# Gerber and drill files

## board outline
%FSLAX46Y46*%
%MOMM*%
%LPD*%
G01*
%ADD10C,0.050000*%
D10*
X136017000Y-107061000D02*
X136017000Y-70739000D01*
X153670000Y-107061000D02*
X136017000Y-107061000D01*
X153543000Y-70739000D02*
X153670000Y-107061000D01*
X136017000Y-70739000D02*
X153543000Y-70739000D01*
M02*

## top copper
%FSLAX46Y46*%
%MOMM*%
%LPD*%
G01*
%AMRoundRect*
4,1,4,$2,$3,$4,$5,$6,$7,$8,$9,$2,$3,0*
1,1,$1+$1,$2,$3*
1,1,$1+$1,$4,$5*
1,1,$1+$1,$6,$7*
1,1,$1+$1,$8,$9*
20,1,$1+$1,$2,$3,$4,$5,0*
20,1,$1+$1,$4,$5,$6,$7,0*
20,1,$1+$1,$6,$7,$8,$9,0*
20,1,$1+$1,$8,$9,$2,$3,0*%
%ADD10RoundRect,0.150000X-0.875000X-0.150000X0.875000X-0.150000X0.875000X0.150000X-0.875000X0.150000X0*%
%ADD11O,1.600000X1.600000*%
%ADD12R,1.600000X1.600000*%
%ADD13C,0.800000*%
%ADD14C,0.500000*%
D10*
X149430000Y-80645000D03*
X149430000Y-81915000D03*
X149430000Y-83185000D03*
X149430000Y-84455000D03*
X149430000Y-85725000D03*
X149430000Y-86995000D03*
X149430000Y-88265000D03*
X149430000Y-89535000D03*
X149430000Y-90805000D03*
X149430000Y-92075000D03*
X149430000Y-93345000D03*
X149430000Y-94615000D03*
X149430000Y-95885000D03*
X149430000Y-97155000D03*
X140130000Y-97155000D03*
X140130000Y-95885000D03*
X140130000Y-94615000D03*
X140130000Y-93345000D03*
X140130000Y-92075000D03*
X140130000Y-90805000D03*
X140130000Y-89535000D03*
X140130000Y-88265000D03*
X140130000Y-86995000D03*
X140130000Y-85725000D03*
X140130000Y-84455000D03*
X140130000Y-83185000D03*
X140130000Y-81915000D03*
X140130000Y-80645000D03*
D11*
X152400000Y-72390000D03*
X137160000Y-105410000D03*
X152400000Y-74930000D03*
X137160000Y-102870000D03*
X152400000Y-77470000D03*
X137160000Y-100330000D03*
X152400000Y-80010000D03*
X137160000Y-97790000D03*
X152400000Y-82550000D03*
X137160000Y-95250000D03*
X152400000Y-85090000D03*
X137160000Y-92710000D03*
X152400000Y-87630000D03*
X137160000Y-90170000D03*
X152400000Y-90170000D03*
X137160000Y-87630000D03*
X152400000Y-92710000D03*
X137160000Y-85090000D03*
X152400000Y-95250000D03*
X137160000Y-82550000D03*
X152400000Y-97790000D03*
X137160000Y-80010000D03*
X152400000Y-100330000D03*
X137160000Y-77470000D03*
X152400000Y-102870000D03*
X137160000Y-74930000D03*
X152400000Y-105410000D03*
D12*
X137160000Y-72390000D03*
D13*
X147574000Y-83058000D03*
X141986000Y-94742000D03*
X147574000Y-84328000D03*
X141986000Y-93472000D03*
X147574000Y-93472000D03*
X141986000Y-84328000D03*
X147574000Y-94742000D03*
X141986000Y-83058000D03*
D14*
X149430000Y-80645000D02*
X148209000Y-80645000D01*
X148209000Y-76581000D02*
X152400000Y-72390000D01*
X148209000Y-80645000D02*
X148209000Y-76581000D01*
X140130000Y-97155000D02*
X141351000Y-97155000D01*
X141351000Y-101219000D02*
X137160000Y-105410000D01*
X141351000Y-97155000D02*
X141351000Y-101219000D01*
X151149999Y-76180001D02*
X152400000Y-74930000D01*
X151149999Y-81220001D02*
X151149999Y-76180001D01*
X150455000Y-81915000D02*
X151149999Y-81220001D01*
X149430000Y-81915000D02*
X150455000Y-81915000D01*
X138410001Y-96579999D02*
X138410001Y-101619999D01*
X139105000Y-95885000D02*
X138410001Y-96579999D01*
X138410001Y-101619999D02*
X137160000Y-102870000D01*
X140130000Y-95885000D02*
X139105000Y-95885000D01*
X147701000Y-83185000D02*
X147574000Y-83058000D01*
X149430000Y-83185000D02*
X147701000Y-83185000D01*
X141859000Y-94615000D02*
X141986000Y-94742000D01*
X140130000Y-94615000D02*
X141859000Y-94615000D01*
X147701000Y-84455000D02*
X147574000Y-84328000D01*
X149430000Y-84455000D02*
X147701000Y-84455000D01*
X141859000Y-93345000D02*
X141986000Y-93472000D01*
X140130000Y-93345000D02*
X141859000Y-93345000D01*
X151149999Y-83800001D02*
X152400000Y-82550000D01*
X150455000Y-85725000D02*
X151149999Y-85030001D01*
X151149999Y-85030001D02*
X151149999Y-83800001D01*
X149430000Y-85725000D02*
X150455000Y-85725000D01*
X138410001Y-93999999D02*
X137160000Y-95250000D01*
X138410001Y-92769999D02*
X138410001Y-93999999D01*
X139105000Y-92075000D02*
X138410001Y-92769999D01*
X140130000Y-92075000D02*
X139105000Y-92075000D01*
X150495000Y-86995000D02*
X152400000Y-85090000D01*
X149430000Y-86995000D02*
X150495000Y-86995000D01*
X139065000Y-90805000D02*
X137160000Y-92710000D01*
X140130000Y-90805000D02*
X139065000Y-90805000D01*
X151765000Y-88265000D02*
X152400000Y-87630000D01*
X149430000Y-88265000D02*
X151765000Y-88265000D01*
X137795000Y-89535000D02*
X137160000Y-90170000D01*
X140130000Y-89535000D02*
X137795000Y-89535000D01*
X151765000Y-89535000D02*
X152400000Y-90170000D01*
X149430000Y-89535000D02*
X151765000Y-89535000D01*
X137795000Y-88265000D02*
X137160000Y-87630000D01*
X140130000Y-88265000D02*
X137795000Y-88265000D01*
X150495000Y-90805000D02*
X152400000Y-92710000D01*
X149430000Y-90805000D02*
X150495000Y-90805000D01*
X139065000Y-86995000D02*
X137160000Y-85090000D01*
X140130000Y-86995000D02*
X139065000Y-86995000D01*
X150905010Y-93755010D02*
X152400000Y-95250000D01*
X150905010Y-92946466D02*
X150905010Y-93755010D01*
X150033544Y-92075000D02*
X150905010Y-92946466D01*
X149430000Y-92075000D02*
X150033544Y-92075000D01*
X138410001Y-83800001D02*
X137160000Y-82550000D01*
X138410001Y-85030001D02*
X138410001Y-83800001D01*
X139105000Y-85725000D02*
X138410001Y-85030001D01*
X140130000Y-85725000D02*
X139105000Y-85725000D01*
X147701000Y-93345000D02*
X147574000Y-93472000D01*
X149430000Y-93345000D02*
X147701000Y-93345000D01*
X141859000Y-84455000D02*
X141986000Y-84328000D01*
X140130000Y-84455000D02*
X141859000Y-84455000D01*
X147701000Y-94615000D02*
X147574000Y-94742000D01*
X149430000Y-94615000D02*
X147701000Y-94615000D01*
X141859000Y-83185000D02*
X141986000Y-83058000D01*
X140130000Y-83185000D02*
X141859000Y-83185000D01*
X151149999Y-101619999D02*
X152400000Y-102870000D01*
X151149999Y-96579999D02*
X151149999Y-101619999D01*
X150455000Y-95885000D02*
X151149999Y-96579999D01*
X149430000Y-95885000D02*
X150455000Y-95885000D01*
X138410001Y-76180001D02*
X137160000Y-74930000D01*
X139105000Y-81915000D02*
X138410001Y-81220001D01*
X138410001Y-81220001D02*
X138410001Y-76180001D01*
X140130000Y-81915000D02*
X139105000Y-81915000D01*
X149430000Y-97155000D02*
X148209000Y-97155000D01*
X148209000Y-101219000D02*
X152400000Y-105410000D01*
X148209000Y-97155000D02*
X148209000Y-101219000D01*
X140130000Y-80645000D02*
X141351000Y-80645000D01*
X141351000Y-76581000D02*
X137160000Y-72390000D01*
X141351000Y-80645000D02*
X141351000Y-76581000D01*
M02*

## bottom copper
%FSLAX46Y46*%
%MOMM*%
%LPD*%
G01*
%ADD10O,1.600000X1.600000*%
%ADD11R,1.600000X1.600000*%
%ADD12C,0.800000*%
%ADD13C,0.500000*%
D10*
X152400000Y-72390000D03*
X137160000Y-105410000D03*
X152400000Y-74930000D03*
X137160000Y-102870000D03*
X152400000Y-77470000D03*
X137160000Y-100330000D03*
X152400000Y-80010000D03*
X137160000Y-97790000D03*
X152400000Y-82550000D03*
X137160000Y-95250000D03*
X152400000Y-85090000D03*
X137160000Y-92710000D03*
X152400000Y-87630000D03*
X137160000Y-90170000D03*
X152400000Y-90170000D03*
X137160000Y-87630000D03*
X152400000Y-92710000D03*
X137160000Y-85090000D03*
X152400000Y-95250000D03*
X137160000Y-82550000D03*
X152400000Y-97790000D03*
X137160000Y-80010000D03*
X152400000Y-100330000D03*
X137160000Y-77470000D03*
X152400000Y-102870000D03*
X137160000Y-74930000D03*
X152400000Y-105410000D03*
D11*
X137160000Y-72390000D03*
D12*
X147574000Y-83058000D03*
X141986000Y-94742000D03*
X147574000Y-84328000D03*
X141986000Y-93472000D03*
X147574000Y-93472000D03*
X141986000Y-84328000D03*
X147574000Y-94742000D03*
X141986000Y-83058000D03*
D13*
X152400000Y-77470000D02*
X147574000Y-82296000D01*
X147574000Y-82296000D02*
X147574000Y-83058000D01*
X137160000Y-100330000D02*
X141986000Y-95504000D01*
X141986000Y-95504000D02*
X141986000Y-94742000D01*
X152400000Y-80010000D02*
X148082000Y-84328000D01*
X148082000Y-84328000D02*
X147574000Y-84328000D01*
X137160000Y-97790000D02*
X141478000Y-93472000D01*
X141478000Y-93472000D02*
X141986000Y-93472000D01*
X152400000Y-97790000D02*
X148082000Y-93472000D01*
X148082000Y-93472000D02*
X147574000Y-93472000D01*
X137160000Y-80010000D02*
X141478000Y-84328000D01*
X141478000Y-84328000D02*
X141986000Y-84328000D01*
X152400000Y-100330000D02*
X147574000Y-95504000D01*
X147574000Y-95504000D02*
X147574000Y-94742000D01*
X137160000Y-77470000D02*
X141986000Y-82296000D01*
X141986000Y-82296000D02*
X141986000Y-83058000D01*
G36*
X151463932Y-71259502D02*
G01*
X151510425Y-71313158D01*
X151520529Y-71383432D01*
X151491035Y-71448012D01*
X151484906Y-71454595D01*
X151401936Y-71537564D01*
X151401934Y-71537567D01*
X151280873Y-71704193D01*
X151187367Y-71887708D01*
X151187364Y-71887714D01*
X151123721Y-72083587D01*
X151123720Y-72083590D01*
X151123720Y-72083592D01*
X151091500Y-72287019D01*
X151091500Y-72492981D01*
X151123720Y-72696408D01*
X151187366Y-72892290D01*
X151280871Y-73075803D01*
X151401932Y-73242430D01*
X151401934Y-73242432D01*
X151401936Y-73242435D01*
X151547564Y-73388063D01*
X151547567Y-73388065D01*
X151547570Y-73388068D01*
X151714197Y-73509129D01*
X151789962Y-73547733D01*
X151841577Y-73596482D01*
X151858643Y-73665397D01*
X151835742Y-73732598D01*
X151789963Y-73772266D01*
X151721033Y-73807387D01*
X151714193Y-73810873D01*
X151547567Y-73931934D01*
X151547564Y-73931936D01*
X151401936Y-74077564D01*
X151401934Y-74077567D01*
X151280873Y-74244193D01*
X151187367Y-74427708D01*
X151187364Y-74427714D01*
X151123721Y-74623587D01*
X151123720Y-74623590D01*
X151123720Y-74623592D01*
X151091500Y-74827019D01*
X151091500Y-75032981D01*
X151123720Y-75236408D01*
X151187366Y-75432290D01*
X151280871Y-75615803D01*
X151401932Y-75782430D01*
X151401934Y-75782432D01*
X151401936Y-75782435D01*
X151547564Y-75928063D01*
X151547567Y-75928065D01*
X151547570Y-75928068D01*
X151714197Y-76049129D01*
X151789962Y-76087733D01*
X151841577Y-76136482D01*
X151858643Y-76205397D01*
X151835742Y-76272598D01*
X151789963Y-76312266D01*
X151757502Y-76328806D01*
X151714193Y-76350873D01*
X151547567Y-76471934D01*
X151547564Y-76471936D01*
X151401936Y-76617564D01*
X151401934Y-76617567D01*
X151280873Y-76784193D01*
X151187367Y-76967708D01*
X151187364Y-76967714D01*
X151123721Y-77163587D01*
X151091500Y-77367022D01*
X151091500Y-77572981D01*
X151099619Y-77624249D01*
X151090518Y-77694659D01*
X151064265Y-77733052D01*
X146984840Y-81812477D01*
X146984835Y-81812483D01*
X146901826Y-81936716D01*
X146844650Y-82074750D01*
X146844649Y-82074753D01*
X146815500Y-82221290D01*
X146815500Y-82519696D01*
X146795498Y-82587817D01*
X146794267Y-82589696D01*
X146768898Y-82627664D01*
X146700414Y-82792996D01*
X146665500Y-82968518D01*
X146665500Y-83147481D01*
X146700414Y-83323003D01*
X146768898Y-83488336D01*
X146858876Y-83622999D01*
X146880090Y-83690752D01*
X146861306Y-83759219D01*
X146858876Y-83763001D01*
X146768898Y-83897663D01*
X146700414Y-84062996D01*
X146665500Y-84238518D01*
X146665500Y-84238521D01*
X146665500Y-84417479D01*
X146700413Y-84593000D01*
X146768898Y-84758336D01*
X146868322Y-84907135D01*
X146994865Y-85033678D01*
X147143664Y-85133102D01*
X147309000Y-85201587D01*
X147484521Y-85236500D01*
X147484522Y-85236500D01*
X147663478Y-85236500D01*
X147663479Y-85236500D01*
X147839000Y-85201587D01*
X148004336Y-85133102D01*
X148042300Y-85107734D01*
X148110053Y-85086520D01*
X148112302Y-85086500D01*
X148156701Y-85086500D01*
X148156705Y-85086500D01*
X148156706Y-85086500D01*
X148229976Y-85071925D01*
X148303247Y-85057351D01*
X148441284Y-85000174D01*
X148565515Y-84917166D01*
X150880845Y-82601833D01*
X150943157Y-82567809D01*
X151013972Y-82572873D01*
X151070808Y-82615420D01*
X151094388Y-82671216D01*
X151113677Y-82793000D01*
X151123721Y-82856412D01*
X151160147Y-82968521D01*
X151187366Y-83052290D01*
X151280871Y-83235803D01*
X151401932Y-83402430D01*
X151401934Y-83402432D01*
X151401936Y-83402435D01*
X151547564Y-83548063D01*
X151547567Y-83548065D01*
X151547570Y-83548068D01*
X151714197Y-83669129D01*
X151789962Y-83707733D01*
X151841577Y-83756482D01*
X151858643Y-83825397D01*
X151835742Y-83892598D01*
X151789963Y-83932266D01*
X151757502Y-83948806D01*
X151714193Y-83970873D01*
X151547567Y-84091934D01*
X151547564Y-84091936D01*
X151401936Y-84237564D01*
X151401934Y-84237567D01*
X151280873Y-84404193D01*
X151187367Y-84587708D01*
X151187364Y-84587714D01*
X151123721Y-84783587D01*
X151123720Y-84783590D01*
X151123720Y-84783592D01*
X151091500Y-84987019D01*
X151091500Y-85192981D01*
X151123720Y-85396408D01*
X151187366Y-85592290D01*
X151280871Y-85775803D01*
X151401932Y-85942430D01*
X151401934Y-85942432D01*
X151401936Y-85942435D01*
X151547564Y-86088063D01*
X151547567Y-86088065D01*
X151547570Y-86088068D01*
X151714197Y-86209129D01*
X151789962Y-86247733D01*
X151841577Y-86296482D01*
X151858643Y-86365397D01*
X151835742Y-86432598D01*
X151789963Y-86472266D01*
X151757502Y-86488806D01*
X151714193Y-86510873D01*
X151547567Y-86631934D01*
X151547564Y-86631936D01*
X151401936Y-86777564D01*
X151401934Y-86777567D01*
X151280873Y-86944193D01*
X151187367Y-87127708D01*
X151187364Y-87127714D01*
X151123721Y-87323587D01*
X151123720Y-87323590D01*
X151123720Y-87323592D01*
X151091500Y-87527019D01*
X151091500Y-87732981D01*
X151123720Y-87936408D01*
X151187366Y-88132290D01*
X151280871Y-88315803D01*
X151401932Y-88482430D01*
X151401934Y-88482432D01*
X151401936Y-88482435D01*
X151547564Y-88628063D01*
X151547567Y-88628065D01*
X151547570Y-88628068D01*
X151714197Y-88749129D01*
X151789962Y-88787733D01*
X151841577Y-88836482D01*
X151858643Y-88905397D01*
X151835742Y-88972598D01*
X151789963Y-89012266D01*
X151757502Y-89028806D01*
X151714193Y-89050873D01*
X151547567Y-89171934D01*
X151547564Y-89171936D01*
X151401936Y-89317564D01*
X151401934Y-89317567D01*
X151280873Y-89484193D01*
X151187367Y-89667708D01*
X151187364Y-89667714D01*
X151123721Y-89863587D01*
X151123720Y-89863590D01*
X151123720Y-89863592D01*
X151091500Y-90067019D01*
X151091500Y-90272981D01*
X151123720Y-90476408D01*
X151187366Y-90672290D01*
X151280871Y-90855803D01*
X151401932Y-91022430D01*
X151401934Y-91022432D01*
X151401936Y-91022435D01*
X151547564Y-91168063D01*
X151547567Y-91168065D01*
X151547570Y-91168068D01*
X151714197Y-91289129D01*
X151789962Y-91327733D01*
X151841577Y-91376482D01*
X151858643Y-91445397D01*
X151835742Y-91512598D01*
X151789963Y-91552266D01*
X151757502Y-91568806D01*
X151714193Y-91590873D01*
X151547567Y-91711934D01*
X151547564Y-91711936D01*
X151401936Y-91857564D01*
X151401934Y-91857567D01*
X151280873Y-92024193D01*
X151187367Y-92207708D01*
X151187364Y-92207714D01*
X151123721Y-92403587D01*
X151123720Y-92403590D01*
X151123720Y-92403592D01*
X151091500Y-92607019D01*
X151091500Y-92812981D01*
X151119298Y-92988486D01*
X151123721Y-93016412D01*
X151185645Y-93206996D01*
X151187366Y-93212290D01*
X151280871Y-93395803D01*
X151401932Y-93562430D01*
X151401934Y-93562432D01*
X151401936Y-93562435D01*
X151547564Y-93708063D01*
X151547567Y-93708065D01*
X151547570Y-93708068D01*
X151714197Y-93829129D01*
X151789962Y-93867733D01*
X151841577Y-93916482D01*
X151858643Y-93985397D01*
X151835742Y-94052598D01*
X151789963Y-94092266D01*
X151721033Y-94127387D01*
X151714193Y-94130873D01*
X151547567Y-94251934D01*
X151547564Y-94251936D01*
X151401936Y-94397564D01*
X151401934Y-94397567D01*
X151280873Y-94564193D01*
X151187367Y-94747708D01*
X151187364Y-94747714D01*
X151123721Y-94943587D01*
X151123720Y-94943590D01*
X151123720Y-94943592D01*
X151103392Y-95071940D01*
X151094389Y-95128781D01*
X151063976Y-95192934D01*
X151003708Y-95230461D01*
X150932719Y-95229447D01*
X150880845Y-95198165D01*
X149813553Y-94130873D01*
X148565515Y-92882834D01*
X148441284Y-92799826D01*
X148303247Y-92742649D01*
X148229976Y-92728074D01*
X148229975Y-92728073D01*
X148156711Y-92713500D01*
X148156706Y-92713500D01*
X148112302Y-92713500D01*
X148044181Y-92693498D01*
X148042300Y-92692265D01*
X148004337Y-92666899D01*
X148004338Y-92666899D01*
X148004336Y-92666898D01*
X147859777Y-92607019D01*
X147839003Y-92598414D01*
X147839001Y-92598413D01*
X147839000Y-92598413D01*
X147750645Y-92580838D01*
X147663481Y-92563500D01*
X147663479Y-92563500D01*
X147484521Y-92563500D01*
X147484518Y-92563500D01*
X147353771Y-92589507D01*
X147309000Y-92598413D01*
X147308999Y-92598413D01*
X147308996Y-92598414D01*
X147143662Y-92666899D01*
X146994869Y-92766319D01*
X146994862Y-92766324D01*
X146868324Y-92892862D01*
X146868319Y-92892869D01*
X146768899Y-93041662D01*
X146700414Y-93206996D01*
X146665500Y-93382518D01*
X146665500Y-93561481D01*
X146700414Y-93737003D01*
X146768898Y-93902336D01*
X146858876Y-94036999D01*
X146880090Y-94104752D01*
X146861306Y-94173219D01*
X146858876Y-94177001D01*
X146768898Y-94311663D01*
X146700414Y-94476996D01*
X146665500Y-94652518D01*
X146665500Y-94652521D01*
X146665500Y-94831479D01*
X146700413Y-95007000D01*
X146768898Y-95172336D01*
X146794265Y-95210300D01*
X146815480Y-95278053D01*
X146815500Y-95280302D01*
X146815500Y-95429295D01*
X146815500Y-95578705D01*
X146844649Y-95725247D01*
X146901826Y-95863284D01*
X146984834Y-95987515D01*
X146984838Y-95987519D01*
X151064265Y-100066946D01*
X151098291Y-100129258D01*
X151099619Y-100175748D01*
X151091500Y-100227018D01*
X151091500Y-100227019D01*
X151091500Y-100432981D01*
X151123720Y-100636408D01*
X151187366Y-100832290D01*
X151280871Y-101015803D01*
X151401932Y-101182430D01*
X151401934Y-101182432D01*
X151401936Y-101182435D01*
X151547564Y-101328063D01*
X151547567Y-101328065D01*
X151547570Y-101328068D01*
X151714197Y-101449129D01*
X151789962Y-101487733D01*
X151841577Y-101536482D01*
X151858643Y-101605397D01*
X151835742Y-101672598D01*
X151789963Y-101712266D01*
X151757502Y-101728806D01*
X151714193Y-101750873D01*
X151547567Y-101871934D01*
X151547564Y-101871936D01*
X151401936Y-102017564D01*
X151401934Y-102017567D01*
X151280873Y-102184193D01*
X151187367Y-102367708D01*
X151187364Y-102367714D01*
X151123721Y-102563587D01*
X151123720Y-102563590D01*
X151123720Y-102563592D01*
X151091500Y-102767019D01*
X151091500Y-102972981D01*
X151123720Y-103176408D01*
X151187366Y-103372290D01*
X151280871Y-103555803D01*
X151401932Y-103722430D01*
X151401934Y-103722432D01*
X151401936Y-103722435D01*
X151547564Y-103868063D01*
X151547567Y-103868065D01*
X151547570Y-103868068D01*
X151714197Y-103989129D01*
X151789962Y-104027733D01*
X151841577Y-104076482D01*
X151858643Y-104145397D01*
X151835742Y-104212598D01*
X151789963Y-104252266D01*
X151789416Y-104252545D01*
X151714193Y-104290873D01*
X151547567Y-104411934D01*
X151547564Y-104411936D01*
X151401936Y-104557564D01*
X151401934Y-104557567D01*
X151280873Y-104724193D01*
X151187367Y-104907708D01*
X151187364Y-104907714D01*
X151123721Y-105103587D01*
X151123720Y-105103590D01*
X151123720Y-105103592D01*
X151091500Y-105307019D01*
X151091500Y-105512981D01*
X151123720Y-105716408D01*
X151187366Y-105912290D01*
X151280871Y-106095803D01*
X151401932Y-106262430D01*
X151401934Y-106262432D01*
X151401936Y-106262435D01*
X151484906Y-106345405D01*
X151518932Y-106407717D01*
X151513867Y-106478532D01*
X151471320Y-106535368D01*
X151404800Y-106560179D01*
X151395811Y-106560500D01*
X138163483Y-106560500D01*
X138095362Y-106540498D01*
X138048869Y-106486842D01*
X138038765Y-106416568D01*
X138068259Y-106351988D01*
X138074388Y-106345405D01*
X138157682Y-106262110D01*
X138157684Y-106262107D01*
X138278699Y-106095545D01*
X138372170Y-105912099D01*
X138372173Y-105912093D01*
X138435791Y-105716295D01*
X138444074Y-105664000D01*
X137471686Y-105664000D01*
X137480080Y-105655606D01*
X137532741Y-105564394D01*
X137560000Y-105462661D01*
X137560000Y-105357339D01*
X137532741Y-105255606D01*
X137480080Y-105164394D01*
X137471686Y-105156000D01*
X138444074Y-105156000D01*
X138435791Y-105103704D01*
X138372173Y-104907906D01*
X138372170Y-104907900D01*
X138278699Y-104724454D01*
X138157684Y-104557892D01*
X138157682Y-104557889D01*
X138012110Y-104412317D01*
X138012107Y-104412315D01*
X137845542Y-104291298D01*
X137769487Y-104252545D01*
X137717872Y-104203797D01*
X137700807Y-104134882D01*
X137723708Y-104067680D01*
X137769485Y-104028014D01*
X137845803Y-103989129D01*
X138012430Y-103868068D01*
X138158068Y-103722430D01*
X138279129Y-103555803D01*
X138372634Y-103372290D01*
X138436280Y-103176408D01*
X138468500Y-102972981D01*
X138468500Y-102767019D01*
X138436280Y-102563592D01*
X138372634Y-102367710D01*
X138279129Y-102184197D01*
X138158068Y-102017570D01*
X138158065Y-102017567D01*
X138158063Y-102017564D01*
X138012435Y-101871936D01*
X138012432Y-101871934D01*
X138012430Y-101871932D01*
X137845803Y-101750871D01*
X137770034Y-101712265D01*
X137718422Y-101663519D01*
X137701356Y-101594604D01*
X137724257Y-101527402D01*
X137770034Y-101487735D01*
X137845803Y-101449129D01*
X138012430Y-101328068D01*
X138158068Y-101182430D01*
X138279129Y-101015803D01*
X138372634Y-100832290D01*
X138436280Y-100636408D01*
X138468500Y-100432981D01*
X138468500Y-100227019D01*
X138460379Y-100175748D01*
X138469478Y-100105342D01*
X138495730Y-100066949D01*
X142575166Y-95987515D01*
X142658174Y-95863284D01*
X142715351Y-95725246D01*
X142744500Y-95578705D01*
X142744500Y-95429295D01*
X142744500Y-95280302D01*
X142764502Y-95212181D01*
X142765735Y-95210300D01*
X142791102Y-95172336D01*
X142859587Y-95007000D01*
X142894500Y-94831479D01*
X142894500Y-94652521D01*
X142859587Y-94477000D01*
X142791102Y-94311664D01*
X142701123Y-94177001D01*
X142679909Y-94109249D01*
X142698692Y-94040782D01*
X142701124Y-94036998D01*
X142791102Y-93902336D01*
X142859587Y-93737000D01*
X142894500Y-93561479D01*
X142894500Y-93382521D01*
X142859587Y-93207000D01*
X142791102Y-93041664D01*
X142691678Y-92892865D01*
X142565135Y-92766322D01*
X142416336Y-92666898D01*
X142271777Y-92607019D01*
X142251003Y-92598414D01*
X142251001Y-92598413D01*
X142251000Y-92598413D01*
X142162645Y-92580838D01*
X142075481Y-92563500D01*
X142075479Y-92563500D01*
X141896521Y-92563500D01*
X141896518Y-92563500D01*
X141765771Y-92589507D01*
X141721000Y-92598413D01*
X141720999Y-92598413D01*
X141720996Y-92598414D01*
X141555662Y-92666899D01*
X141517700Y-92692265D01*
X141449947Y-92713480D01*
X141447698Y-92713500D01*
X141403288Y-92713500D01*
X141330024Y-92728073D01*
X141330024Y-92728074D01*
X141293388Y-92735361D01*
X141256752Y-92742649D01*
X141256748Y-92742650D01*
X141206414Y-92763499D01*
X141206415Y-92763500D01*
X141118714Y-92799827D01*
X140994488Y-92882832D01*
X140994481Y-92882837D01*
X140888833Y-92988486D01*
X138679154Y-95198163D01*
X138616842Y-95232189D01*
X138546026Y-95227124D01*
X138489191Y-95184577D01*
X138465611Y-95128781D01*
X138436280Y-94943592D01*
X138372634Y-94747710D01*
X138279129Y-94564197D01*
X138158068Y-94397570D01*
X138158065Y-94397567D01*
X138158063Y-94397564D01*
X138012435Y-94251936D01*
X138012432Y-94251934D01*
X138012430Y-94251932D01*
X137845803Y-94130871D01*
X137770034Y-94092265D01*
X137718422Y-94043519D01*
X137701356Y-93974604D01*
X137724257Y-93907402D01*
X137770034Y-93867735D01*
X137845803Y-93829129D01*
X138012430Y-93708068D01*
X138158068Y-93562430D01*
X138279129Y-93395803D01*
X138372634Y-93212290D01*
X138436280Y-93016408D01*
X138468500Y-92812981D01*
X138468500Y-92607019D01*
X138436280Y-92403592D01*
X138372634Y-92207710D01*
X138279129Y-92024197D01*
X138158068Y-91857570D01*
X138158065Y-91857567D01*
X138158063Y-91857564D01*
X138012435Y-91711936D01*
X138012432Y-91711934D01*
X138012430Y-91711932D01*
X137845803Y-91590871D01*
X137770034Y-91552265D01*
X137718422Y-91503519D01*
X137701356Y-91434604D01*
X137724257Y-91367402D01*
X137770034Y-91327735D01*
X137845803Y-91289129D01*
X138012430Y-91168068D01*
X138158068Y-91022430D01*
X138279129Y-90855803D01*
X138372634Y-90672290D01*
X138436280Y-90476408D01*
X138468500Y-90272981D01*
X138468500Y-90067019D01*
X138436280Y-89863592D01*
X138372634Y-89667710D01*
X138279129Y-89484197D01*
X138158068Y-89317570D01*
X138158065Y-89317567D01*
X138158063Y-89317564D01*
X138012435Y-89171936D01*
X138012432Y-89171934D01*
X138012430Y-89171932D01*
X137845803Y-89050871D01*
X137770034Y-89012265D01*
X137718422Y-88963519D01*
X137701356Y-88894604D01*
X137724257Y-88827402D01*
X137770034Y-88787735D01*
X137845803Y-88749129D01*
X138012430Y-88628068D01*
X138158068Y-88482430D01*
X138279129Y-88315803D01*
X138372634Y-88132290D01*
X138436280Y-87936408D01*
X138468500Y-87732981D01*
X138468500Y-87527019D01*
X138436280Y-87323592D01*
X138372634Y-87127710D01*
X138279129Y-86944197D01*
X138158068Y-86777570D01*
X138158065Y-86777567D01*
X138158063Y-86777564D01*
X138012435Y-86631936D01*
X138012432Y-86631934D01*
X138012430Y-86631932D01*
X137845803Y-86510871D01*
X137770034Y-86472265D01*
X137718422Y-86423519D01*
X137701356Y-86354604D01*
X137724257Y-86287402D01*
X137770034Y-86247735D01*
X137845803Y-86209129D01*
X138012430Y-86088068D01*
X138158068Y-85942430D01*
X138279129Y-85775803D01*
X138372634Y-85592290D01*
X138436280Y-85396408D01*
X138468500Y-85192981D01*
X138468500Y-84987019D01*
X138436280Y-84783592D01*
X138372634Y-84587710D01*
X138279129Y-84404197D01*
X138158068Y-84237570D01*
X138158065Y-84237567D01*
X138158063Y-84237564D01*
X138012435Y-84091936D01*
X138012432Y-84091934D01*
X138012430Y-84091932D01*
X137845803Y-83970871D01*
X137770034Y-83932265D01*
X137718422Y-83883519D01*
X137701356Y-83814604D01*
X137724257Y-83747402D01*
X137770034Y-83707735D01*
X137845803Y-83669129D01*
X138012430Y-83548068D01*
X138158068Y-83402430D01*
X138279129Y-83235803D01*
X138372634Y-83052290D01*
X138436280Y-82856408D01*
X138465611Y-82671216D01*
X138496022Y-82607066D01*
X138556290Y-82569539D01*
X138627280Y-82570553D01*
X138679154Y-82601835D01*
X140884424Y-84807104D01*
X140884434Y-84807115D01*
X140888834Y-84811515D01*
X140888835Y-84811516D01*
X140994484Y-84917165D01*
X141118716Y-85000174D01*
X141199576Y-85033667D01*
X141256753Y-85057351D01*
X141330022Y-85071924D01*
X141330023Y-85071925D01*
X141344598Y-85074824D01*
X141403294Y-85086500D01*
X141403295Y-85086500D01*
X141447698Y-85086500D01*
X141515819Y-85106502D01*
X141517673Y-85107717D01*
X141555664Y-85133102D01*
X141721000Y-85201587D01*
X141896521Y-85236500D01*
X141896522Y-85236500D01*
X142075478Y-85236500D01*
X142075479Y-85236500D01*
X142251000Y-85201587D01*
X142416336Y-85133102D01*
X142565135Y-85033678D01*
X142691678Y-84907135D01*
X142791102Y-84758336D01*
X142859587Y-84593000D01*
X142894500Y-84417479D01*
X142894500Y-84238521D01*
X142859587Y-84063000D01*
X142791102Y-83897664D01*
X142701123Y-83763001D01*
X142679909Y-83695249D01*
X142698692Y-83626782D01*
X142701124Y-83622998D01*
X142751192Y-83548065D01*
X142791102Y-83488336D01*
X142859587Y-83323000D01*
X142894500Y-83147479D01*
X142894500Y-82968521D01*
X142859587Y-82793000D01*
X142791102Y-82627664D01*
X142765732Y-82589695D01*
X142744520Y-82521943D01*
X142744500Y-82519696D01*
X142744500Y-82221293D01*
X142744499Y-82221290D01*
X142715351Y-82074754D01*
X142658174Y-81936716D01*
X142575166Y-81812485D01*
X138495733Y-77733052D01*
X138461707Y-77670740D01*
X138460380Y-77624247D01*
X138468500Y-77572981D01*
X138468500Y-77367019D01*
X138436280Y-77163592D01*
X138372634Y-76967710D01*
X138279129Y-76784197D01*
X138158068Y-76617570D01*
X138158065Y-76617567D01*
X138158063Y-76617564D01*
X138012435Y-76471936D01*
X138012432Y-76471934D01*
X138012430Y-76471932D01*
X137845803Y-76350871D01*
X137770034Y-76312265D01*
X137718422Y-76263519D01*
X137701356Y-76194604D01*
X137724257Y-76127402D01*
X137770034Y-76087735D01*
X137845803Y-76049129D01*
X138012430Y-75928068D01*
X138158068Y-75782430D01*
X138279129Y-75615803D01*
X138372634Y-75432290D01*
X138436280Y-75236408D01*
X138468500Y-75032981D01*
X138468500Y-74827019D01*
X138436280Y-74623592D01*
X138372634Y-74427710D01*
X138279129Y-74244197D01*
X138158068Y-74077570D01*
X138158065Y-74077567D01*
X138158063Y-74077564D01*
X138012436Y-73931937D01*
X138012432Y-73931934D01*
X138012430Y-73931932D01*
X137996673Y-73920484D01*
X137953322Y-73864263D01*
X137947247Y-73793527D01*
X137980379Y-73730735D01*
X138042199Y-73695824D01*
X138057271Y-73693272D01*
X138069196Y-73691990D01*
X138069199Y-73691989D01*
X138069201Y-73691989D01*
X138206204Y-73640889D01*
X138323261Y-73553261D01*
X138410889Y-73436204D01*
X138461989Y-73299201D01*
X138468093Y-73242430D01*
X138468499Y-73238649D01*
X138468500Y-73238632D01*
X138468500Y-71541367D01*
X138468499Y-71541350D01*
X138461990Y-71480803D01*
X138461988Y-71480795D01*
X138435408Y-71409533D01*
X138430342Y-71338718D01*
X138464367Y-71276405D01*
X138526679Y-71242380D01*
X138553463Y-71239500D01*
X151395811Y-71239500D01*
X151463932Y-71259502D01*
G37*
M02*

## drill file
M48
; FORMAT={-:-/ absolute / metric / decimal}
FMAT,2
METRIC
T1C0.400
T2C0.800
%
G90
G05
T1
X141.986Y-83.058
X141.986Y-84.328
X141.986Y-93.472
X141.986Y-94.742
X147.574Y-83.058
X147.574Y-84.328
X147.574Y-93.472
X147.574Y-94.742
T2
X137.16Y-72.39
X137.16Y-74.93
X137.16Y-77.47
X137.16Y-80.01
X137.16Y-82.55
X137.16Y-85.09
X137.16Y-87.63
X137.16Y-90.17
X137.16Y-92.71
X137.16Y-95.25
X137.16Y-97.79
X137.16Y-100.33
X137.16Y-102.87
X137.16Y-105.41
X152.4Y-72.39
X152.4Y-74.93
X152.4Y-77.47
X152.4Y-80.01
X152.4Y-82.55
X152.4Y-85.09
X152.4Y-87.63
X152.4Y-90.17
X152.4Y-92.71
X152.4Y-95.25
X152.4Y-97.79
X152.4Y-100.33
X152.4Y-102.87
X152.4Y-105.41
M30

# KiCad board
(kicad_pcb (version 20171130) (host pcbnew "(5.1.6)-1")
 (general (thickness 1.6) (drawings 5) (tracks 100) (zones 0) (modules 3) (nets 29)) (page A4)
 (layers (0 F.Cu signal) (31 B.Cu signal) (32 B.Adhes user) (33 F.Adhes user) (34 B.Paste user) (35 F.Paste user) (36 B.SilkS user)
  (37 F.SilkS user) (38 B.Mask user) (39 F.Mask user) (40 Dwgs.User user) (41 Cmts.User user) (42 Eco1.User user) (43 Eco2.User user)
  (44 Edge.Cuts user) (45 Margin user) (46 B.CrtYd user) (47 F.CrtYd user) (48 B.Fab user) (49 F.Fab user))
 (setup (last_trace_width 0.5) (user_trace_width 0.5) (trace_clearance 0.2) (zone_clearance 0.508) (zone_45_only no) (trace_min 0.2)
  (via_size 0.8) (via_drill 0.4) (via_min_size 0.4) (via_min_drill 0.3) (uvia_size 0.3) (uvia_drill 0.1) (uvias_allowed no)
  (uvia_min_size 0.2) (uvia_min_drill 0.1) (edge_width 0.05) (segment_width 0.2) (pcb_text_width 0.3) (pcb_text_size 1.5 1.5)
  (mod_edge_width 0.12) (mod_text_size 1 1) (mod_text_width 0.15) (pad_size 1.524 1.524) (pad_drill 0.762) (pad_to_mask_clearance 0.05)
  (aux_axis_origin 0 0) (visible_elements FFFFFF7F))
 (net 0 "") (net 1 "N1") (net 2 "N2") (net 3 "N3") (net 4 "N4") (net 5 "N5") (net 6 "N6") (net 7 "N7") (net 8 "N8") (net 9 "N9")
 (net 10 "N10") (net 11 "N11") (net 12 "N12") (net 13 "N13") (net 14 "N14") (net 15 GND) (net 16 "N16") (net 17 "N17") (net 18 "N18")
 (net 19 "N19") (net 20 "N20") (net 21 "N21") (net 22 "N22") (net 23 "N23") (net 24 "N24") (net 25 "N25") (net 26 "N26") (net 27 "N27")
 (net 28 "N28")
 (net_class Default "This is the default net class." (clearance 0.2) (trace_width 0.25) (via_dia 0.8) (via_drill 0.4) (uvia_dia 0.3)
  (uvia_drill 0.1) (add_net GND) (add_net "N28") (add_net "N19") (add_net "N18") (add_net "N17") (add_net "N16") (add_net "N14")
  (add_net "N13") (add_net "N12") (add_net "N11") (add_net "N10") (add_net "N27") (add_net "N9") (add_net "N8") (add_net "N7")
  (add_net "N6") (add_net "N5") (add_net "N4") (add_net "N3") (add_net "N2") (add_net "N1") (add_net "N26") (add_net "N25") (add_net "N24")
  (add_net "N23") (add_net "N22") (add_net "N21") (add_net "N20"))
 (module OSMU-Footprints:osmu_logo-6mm (layer F.Cu) (at 144.78 74.549)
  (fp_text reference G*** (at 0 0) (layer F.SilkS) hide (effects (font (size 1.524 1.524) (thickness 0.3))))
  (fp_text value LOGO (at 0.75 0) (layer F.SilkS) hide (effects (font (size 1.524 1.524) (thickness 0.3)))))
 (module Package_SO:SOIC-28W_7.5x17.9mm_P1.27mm (layer F.Cu) (at 144.78 88.9)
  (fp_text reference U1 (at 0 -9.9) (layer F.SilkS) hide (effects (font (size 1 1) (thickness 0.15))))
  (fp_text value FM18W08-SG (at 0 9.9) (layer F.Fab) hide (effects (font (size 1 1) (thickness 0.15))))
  (pad 28 smd roundrect (at 4.65 -8.255) (size 2.05 0.6) (layers F.Cu F.Paste F.Mask) (roundrect_rratio 0.25) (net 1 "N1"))
  (pad 27 smd roundrect (at 4.65 -6.985) (size 2.05 0.6) (layers F.Cu F.Paste F.Mask) (roundrect_rratio 0.25) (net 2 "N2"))
  (pad 26 smd roundrect (at 4.65 -5.715) (size 2.05 0.6) (layers F.Cu F.Paste F.Mask) (roundrect_rratio 0.25) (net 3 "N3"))
  (pad 25 smd roundrect (at 4.65 -4.445) (size 2.05 0.6) (layers F.Cu F.Paste F.Mask) (roundrect_rratio 0.25) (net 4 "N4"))
  (pad 24 smd roundrect (at 4.65 -3.175) (size 2.05 0.6) (layers F.Cu F.Paste F.Mask) (roundrect_rratio 0.25) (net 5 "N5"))
  (pad 23 smd roundrect (at 4.65 -1.905) (size 2.05 0.6) (layers F.Cu F.Paste F.Mask) (roundrect_rratio 0.25) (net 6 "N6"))
  (pad 22 smd roundrect (at 4.65 -0.635) (size 2.05 0.6) (layers F.Cu F.Paste F.Mask) (roundrect_rratio 0.25) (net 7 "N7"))
  (pad 21 smd roundrect (at 4.65 0.635) (size 2.05 0.6) (layers F.Cu F.Paste F.Mask) (roundrect_rratio 0.25) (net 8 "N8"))
  (pad 20 smd roundrect (at 4.65 1.905) (size 2.05 0.6) (layers F.Cu F.Paste F.Mask) (roundrect_rratio 0.25) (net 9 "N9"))
  (pad 19 smd roundrect (at 4.65 3.175) (size 2.05 0.6) (layers F.Cu F.Paste F.Mask) (roundrect_rratio 0.25) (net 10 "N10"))
  (pad 18 smd roundrect (at 4.65 4.445) (size 2.05 0.6) (layers F.Cu F.Paste F.Mask) (roundrect_rratio 0.25) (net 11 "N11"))
  (pad 17 smd roundrect (at 4.65 5.715) (size 2.05 0.6) (layers F.Cu F.Paste F.Mask) (roundrect_rratio 0.25) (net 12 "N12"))
  (pad 16 smd roundrect (at 4.65 6.985) (size 2.05 0.6) (layers F.Cu F.Paste F.Mask) (roundrect_rratio 0.25) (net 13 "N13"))
  (pad 15 smd roundrect (at 4.65 8.255) (size 2.05 0.6) (layers F.Cu F.Paste F.Mask) (roundrect_rratio 0.25) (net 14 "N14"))
  (pad 14 smd roundrect (at -4.65 8.255) (size 2.05 0.6) (layers F.Cu F.Paste F.Mask) (roundrect_rratio 0.25) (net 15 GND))
  (pad 13 smd roundrect (at -4.65 6.985) (size 2.05 0.6) (layers F.Cu F.Paste F.Mask) (roundrect_rratio 0.25) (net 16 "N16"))
  (pad 12 smd roundrect (at -4.65 5.715) (size 2.05 0.6) (layers F.Cu F.Paste F.Mask) (roundrect_rratio 0.25) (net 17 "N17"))
  (pad 11 smd roundrect (at -4.65 4.445) (size 2.05 0.6) (layers F.Cu F.Paste F.Mask) (roundrect_rratio 0.25) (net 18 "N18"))
  (pad 10 smd roundrect (at -4.65 3.175) (size 2.05 0.6) (layers F.Cu F.Paste F.Mask) (roundrect_rratio 0.25) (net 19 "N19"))
  (pad 9 smd roundrect (at -4.65 1.905) (size 2.05 0.6) (layers F.Cu F.Paste F.Mask) (roundrect_rratio 0.25) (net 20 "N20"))
  (pad 8 smd roundrect (at -4.65 0.635) (size 2.05 0.6) (layers F.Cu F.Paste F.Mask) (roundrect_rratio 0.25) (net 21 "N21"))
  (pad 7 smd roundrect (at -4.65 -0.635) (size 2.05 0.6) (layers F.Cu F.Paste F.Mask) (roundrect_rratio 0.25) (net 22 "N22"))
  (pad 6 smd roundrect (at -4.65 -1.905) (size 2.05 0.6) (layers F.Cu F.Paste F.Mask) (roundrect_rratio 0.25) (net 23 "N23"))
  (pad 5 smd roundrect (at -4.65 -3.175) (size 2.05 0.6) (layers F.Cu F.Paste F.Mask) (roundrect_rratio 0.25) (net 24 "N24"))
  (pad 4 smd roundrect (at -4.65 -4.445) (size 2.05 0.6) (layers F.Cu F.Paste F.Mask) (roundrect_rratio 0.25) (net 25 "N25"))
  (pad 3 smd roundrect (at -4.65 -5.715) (size 2.05 0.6) (layers F.Cu F.Paste F.Mask) (roundrect_rratio 0.25) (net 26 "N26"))
  (pad 2 smd roundrect (at -4.65 -6.985) (size 2.05 0.6) (layers F.Cu F.Paste F.Mask) (roundrect_rratio 0.25) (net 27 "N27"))
  (pad 1 smd roundrect (at -4.65 -8.255) (size 2.05 0.6) (layers F.Cu F.Paste F.Mask) (roundrect_rratio 0.25) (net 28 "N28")))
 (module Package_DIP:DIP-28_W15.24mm (layer F.Cu) (at 137.16 72.39)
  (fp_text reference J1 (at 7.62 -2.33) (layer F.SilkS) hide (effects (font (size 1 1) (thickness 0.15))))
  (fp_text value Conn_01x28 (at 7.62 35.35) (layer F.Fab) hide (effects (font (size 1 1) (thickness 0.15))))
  (pad 28 thru_hole oval (at 15.24 0) (size 1.6 1.6) (drill 0.8) (layers *.Cu *.Mask) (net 1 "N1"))
  (pad 14 thru_hole oval (at 0 33.02) (size 1.6 1.6) (drill 0.8) (layers *.Cu *.Mask) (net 15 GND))
  (pad 27 thru_hole oval (at 15.24 2.54) (size 1.6 1.6) (drill 0.8) (layers *.Cu *.Mask) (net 2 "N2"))
  (pad 13 thru_hole oval (at 0 30.48) (size 1.6 1.6) (drill 0.8) (layers *.Cu *.Mask) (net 16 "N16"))
  (pad 26 thru_hole oval (at 15.24 5.08) (size 1.6 1.6) (drill 0.8) (layers *.Cu *.Mask) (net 3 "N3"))
  (pad 12 thru_hole oval (at 0 27.94) (size 1.6 1.6) (drill 0.8) (layers *.Cu *.Mask) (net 17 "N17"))
  (pad 25 thru_hole oval (at 15.24 7.62) (size 1.6 1.6) (drill 0.8) (layers *.Cu *.Mask) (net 4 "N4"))
  (pad 11 thru_hole oval (at 0 25.4) (size 1.6 1.6) (drill 0.8) (layers *.Cu *.Mask) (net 18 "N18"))
  (pad 24 thru_hole oval (at 15.24 10.16) (size 1.6 1.6) (drill 0.8) (layers *.Cu *.Mask) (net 5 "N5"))
  (pad 10 thru_hole oval (at 0 22.86) (size 1.6 1.6) (drill 0.8) (layers *.Cu *.Mask) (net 19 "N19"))
  (pad 23 thru_hole oval (at 15.24 12.7) (size 1.6 1.6) (drill 0.8) (layers *.Cu *.Mask) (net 6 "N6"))
  (pad 9 thru_hole oval (at 0 20.32) (size 1.6 1.6) (drill 0.8) (layers *.Cu *.Mask) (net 20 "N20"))
  (pad 22 thru_hole oval (at 15.24 15.24) (size 1.6 1.6) (drill 0.8) (layers *.Cu *.Mask) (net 7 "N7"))
  (pad 8 thru_hole oval (at 0 17.78) (size 1.6 1.6) (drill 0.8) (layers *.Cu *.Mask) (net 21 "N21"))
  (pad 21 thru_hole oval (at 15.24 17.78) (size 1.6 1.6) (drill 0.8) (layers *.Cu *.Mask) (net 8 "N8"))
  (pad 7 thru_hole oval (at 0 15.24) (size 1.6 1.6) (drill 0.8) (layers *.Cu *.Mask) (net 22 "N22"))
  (pad 20 thru_hole oval (at 15.24 20.32) (size 1.6 1.6) (drill 0.8) (layers *.Cu *.Mask) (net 9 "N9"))
  (pad 6 thru_hole oval (at 0 12.7) (size 1.6 1.6) (drill 0.8) (layers *.Cu *.Mask) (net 23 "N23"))
  (pad 19 thru_hole oval (at 15.24 22.86) (size 1.6 1.6) (drill 0.8) (layers *.Cu *.Mask) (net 10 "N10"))
  (pad 5 thru_hole oval (at 0 10.16) (size 1.6 1.6) (drill 0.8) (layers *.Cu *.Mask) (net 24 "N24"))
  (pad 18 thru_hole oval (at 15.24 25.4) (size 1.6 1.6) (drill 0.8) (layers *.Cu *.Mask) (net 11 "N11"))
  (pad 4 thru_hole oval (at 0 7.62) (size 1.6 1.6) (drill 0.8) (layers *.Cu *.Mask) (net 25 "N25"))
  (pad 17 thru_hole oval (at 15.24 27.94) (size 1.6 1.6) (drill 0.8) (layers *.Cu *.Mask) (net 12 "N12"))
  (pad 3 thru_hole oval (at 0 5.08) (size 1.6 1.6) (drill 0.8) (layers *.Cu *.Mask) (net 26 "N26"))
  (pad 16 thru_hole oval (at 15.24 30.48) (size 1.6 1.6) (drill 0.8) (layers *.Cu *.Mask) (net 13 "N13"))
  (pad 2 thru_hole oval (at 0 2.54) (size 1.6 1.6) (drill 0.8) (layers *.Cu *.Mask) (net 27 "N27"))
  (pad 15 thru_hole oval (at 15.24 33.02) (size 1.6 1.6) (drill 0.8) (layers *.Cu *.Mask) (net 14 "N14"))
  (pad 1 thru_hole rect (at 0 0) (size 1.6 1.6) (drill 0.8) (layers *.Cu *.Mask) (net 28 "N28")))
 (gr_line (start 136.017 107.061) (end 136.017 70.739) (layer Edge.Cuts) (width 0.05))
 (gr_line (start 153.67 107.061) (end 136.017 107.061) (layer Edge.Cuts) (width 0.05))
 (gr_line (start 153.543 70.739) (end 153.67 107.061) (layer Edge.Cuts) (width 0.05))
 (gr_line (start 136.017 70.739) (end 153.543 70.739) (layer Edge.Cuts) (width 0.05))
 (segment (start 149.43 80.645) (end 148.209 80.645) (width 0.5) (layer F.Cu) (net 1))
 (segment (start 148.209 76.581) (end 152.4 72.39) (width 0.5) (layer F.Cu) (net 1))
 (segment (start 148.209 80.645) (end 148.209 76.581) (width 0.5) (layer F.Cu) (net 1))
 (segment (start 140.13 97.155) (end 141.351 97.155) (width 0.5) (layer F.Cu) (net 15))
 (segment (start 141.351 101.219) (end 137.16 105.41) (width 0.5) (layer F.Cu) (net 15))
 (segment (start 141.351 97.155) (end 141.351 101.219) (width 0.5) (layer F.Cu) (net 15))
 (segment (start 151.149999 76.180001) (end 152.4 74.93) (width 0.5) (layer F.Cu) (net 2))
 (segment (start 151.149999 81.220001) (end 151.149999 76.180001) (width 0.5) (layer F.Cu) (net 2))
 (segment (start 150.455 81.915) (end 151.149999 81.220001) (width 0.5) (layer F.Cu) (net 2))
 (segment (start 149.43 81.915) (end 150.455 81.915) (width 0.5) (layer F.Cu) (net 2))
 (segment (start 138.410001 96.579999) (end 138.410001 101.619999) (width 0.5) (layer F.Cu) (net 16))
 (segment (start 139.105 95.885) (end 138.410001 96.579999) (width 0.5) (layer F.Cu) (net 16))
 (segment (start 138.410001 101.619999) (end 137.16 102.87) (width 0.5) (layer F.Cu) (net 16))
 (segment (start 140.13 95.885) (end 139.105 95.885) (width 0.5) (layer F.Cu) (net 16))
 (via (at 147.574 83.058) (size 0.8) (drill 0.4) (layers F.Cu B.Cu) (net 3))
 (segment (start 152.4 77.47) (end 147.574 82.296) (width 0.5) (layer B.Cu) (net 3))
 (segment (start 147.574 82.296) (end 147.574 83.058) (width 0.5) (layer B.Cu) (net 3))
 (segment (start 147.701 83.185) (end 147.574 83.058) (width 0.5) (layer F.Cu) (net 3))
 (segment (start 149.43 83.185) (end 147.701 83.185) (width 0.5) (layer F.Cu) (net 3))
 (via (at 141.986 94.742) (size 0.8) (drill 0.4) (layers F.Cu B.Cu) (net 17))
 (segment (start 137.16 100.33) (end 141.986 95.504) (width 0.5) (layer B.Cu) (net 17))
 (segment (start 141.986 95.504) (end 141.986 94.742) (width 0.5) (layer B.Cu) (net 17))
 (segment (start 141.859 94.615) (end 141.986 94.742) (width 0.5) (layer F.Cu) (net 17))
 (segment (start 140.13 94.615) (end 141.859 94.615) (width 0.5) (layer F.Cu) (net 17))
 (via (at 147.574 84.328) (size 0.8) (drill 0.4) (layers F.Cu B.Cu) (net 4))
 (segment (start 152.4 80.01) (end 148.082 84.328) (width 0.5) (layer B.Cu) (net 4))
 (segment (start 147.701 84.455) (end 147.574 84.328) (width 0.5) (layer F.Cu) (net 4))
 (segment (start 149.43 84.455) (end 147.701 84.455) (width 0.5) (layer F.Cu) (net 4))
 (segment (start 148.082 84.328) (end 147.574 84.328) (width 0.5) (layer B.Cu) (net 4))
 (via (at 141.986 93.472) (size 0.8) (drill 0.4) (layers F.Cu B.Cu) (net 18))
 (segment (start 137.16 97.79) (end 141.478 93.472) (width 0.5) (layer B.Cu) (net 18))
 (segment (start 141.478 93.472) (end 141.986 93.472) (width 0.5) (layer B.Cu) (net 18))
 (segment (start 141.859 93.345) (end 141.986 93.472) (width 0.5) (layer F.Cu) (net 18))
 (segment (start 140.13 93.345) (end 141.859 93.345) (width 0.5) (layer F.Cu) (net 18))
 (segment (start 151.149999 83.800001) (end 152.4 82.55) (width 0.5) (layer F.Cu) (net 5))
 (segment (start 150.455 85.725) (end 151.149999 85.030001) (width 0.5) (layer F.Cu) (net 5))
 (segment (start 151.149999 85.030001) (end 151.149999 83.800001) (width 0.5) (layer F.Cu) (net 5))
 (segment (start 149.43 85.725) (end 150.455 85.725) (width 0.5) (layer F.Cu) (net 5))
 (segment (start 138.410001 93.999999) (end 137.16 95.25) (width 0.5) (layer F.Cu) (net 19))
 (segment (start 138.410001 92.769999) (end 138.410001 93.999999) (width 0.5) (layer F.Cu) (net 19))
 (segment (start 139.105 92.075) (end 138.410001 92.769999) (width 0.5) (layer F.Cu) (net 19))
 (segment (start 140.13 92.075) (end 139.105 92.075) (width 0.5) (layer F.Cu) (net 19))
 (segment (start 150.495 86.995) (end 152.4 85.09) (width 0.5) (layer F.Cu) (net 6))
 (segment (start 149.43 86.995) (end 150.495 86.995) (width 0.5) (layer F.Cu) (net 6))
 (segment (start 139.065 90.805) (end 137.16 92.71) (width 0.5) (layer F.Cu) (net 20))
 (segment (start 140.13 90.805) (end 139.065 90.805) (width 0.5) (layer F.Cu) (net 20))
 (segment (start 151.765 88.265) (end 152.4 87.63) (width 0.5) (layer F.Cu) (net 7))
 (segment (start 149.43 88.265) (end 151.765 88.265) (width 0.5) (layer F.Cu) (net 7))
 (segment (start 137.795 89.535) (end 137.16 90.17) (width 0.5) (layer F.Cu) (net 21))
 (segment (start 140.13 89.535) (end 137.795 89.535) (width 0.5) (layer F.Cu) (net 21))
 (segment (start 151.765 89.535) (end 152.4 90.17) (width 0.5) (layer F.Cu) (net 8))
 (segment (start 149.43 89.535) (end 151.765 89.535) (width 0.5) (layer F.Cu) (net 8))
 (segment (start 137.795 88.265) (end 137.16 87.63) (width 0.5) (layer F.Cu) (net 22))
 (segment (start 140.13 88.265) (end 137.795 88.265) (width 0.5) (layer F.Cu) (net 22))
 (segment (start 150.495 90.805) (end 152.4 92.71) (width 0.5) (layer F.Cu) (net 9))
 (segment (start 149.43 90.805) (end 150.495 90.805) (width 0.5) (layer F.Cu) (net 9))
 (segment (start 139.065 86.995) (end 137.16 85.09) (width 0.5) (layer F.Cu) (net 23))
 (segment (start 140.13 86.995) (end 139.065 86.995) (width 0.5) (layer F.Cu) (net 23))
 (segment (start 150.90501 93.75501) (end 152.4 95.25) (width 0.5) (layer F.Cu) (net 10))
 (segment (start 150.90501 92.946466) (end 150.90501 93.75501) (width 0.5) (layer F.Cu) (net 10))
 (segment (start 150.033544 92.075) (end 150.90501 92.946466) (width 0.5) (layer F.Cu) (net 10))
 (segment (start 149.43 92.075) (end 150.033544 92.075) (width 0.5) (layer F.Cu) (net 10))
 (segment (start 138.410001 83.800001) (end 137.16 82.55) (width 0.5) (layer F.Cu) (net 24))
 (segment (start 138.410001 85.030001) (end 138.410001 83.800001) (width 0.5) (layer F.Cu) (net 24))
 (segment (start 139.105 85.725) (end 138.410001 85.030001) (width 0.5) (layer F.Cu) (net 24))
 (segment (start 140.13 85.725) (end 139.105 85.725) (width 0.5) (layer F.Cu) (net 24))
 (via (at 147.574 93.472) (size 0.8) (drill 0.4) (layers F.Cu B.Cu) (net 11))
 (segment (start 152.4 97.79) (end 148.082 93.472) (width 0.5) (layer B.Cu) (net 11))
 (segment (start 148.082 93.472) (end 147.574 93.472) (width 0.5) (layer B.Cu) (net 11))
 (segment (start 147.701 93.345) (end 147.574 93.472) (width 0.5) (layer F.Cu) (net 11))
 (segment (start 149.43 93.345) (end 147.701 93.345) (width 0.5) (layer F.Cu) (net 11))
 (via (at 141.986 84.328) (size 0.8) (drill 0.4) (layers F.Cu B.Cu) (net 25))
 (segment (start 137.16 80.01) (end 141.478 84.328) (width 0.5) (layer B.Cu) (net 25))
 (segment (start 141.478 84.328) (end 141.986 84.328) (width 0.5) (layer B.Cu) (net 25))
 (segment (start 141.859 84.455) (end 141.986 84.328) (width 0.5) (layer F.Cu) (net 25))
 (segment (start 140.13 84.455) (end 141.859 84.455) (width 0.5) (layer F.Cu) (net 25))
 (via (at 147.574 94.742) (size 0.8) (drill 0.4) (layers F.Cu B.Cu) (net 12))
 (segment (start 152.4 100.33) (end 147.574 95.504) (width 0.5) (layer B.Cu) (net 12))
 (segment (start 147.574 95.504) (end 147.574 94.742) (width 0.5) (layer B.Cu) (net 12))
 (segment (start 147.701 94.615) (end 147.574 94.742) (width 0.5) (layer F.Cu) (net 12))
 (segment (start 149.43 94.615) (end 147.701 94.615) (width 0.5) (layer F.Cu) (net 12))
 (via (at 141.986 83.058) (size 0.8) (drill 0.4) (layers F.Cu B.Cu) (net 26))
 (segment (start 137.16 77.47) (end 141.986 82.296) (width 0.5) (layer B.Cu) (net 26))
 (segment (start 141.986 82.296) (end 141.986 83.058) (width 0.5) (layer B.Cu) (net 26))
 (segment (start 141.859 83.185) (end 141.986 83.058) (width 0.5) (layer F.Cu) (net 26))
 (segment (start 140.13 83.185) (end 141.859 83.185) (width 0.5) (layer F.Cu) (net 26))
 (segment (start 151.149999 101.619999) (end 152.4 102.87) (width 0.5) (layer F.Cu) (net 13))
 (segment (start 151.149999 96.579999) (end 151.149999 101.619999) (width 0.5) (layer F.Cu) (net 13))
 (segment (start 150.455 95.885) (end 151.149999 96.579999) (width 0.5) (layer F.Cu) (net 13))
 (segment (start 149.43 95.885) (end 150.455 95.885) (width 0.5) (layer F.Cu) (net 13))
 (segment (start 138.410001 76.180001) (end 137.16 74.93) (width 0.5) (layer F.Cu) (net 27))
 (segment (start 139.105 81.915) (end 138.410001 81.220001) (width 0.5) (layer F.Cu) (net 27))
 (segment (start 138.410001 81.220001) (end 138.410001 76.180001) (width 0.5) (layer F.Cu) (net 27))
 (segment (start 140.13 81.915) (end 139.105 81.915) (width 0.5) (layer F.Cu) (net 27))
 (segment (start 149.43 97.155) (end 148.209 97.155) (width 0.5) (layer F.Cu) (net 14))
 (segment (start 148.209 101.219) (end 152.4 105.41) (width 0.5) (layer F.Cu) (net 14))
 (segment (start 148.209 97.155) (end 148.209 101.219) (width 0.5) (layer F.Cu) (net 14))
 (segment (start 140.13 80.645) (end 141.351 80.645) (width 0.5) (layer F.Cu) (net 28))
 (segment (start 141.351 76.581) (end 137.16 72.39) (width 0.5) (layer F.Cu) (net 28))
 (segment (start 141.351 80.645) (end 141.351 76.581) (width 0.5) (layer F.Cu) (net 28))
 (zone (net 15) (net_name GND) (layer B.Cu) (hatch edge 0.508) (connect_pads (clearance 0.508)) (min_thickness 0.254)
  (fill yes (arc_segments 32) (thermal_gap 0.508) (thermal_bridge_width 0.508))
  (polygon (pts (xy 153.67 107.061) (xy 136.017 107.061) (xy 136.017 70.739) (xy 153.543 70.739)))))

